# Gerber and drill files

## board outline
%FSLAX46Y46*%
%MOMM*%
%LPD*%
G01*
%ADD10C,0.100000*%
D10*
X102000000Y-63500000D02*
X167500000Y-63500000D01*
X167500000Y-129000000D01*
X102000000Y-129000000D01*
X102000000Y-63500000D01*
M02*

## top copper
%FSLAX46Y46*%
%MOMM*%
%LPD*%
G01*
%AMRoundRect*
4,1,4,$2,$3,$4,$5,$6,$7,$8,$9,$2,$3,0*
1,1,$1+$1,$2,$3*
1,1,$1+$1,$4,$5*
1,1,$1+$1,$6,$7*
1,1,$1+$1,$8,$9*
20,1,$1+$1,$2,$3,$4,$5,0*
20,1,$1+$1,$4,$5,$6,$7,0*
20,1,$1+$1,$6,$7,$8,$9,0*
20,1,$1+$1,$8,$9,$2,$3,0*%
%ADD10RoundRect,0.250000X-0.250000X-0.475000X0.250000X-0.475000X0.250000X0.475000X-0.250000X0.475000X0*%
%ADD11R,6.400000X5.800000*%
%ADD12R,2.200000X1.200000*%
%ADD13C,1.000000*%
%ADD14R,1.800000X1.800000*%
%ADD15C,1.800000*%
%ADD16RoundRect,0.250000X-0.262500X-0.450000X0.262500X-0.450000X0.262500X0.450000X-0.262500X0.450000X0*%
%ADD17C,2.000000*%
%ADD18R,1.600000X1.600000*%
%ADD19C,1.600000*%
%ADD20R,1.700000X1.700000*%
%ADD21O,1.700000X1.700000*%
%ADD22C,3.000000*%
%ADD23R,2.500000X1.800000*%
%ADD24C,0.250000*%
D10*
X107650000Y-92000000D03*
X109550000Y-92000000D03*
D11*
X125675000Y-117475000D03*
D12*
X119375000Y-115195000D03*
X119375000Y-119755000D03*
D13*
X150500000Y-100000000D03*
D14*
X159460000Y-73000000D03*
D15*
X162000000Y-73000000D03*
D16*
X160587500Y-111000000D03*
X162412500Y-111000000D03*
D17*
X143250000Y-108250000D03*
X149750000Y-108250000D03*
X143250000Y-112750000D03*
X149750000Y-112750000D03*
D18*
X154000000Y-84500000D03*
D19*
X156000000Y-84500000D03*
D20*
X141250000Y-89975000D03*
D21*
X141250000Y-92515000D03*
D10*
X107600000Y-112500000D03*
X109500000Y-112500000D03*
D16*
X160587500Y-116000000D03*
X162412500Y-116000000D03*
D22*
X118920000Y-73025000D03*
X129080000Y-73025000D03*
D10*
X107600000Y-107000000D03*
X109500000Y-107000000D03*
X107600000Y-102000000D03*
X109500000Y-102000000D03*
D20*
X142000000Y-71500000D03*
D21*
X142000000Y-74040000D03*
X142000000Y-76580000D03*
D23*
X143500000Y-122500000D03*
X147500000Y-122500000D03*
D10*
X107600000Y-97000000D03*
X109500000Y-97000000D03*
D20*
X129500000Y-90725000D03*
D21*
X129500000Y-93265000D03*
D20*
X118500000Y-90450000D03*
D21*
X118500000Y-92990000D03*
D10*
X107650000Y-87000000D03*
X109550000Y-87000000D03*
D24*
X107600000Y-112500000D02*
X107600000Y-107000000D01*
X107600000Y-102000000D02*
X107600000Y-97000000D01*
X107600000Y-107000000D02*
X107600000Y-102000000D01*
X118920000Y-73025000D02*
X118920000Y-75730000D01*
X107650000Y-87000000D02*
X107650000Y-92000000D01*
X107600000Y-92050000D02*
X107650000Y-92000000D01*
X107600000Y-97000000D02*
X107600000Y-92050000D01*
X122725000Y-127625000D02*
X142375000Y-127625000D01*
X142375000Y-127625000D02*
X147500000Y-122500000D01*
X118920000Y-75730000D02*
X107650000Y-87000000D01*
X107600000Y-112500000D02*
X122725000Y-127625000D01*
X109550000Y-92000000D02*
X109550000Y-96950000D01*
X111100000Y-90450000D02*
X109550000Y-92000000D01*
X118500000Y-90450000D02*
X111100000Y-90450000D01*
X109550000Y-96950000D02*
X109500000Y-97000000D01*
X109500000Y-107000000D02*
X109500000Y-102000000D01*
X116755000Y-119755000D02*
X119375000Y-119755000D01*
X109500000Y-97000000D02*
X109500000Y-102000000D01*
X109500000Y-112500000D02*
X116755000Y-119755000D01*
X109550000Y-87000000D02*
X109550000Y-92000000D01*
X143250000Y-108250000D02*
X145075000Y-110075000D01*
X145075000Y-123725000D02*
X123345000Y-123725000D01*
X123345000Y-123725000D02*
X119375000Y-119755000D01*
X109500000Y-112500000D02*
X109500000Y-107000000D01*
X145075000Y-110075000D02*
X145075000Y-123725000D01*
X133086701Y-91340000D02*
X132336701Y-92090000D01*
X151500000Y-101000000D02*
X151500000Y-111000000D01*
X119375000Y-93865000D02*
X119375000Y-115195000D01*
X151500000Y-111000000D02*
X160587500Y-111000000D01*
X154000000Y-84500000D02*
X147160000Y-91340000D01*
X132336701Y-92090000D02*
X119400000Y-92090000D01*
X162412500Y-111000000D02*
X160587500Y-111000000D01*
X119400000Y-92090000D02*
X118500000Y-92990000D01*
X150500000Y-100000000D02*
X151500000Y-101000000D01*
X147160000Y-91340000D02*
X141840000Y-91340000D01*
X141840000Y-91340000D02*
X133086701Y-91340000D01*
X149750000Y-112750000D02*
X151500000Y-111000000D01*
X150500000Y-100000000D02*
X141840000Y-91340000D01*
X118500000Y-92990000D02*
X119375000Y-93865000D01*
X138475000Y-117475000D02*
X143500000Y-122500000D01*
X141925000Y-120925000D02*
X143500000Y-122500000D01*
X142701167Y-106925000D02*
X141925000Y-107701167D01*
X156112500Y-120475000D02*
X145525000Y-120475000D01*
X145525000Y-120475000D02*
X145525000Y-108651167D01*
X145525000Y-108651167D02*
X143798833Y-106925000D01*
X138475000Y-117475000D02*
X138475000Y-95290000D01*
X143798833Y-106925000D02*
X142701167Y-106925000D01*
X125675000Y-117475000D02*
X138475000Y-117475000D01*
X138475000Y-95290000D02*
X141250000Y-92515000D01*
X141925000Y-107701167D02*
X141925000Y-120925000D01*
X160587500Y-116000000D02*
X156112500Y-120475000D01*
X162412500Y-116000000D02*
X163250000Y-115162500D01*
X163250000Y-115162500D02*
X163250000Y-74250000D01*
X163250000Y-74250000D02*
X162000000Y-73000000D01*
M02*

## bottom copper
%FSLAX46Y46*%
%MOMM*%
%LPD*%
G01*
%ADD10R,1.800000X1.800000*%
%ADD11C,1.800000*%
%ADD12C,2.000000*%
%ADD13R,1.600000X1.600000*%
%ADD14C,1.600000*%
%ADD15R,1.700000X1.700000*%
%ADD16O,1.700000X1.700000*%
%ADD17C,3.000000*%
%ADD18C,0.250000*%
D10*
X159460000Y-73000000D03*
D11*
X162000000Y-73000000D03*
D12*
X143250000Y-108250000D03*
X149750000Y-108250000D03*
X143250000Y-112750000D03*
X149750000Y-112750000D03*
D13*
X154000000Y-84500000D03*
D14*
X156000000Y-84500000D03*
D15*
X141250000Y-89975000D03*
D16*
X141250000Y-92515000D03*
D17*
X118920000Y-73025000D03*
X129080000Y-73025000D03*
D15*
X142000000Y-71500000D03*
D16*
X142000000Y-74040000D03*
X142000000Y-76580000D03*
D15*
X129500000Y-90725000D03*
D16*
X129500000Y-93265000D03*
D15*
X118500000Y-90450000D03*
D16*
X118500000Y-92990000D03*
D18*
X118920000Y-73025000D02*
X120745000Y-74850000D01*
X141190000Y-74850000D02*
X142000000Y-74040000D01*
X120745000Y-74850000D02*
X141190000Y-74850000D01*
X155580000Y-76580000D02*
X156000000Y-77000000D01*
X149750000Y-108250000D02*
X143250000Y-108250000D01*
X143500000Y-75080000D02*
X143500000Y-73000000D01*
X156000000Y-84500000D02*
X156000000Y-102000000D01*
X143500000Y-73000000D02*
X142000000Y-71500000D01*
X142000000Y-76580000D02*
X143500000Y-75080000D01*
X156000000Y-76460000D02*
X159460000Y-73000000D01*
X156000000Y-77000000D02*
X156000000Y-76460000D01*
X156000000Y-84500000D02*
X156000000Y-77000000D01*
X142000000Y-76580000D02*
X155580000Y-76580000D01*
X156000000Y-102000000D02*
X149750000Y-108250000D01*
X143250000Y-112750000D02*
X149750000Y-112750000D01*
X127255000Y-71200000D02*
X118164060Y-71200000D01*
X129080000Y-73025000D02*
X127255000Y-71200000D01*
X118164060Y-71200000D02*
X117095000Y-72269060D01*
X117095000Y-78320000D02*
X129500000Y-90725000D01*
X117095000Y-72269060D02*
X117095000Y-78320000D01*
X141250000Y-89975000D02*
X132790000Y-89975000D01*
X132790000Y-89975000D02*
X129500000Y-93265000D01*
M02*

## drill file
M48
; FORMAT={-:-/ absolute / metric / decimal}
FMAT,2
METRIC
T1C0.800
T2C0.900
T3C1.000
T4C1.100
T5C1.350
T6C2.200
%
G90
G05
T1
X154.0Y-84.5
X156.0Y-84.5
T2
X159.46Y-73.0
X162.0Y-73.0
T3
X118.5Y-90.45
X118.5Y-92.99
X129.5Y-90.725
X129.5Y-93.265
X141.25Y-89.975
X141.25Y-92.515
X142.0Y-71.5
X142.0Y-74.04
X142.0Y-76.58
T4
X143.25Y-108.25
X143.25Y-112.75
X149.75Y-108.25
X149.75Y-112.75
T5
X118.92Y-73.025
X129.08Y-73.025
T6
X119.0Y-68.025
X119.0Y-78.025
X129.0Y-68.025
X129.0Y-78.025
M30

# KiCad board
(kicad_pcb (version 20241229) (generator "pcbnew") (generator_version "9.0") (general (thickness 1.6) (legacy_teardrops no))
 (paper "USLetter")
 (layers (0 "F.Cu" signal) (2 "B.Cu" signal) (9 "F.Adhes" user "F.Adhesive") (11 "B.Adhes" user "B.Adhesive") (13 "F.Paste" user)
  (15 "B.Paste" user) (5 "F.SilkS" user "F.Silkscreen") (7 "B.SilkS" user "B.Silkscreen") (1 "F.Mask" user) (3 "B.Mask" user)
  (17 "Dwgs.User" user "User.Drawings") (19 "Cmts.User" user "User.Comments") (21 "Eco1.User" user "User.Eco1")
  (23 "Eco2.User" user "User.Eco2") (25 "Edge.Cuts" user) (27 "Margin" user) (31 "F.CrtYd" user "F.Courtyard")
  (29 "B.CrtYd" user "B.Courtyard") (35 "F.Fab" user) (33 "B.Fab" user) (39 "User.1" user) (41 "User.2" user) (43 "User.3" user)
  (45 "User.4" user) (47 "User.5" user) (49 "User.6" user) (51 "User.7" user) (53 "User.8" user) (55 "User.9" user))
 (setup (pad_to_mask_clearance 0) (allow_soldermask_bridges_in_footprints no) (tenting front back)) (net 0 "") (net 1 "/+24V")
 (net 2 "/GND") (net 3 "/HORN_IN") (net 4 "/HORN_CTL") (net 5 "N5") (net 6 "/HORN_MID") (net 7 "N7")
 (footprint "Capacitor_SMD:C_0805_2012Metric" (layer "F.Cu") (at 108.6 92)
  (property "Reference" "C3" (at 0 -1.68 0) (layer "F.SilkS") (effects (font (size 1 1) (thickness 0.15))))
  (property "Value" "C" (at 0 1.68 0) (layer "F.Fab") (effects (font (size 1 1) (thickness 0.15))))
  (pad "1" smd roundrect (at -0.95 0) (size 1 1.45) (layers "F.Cu" "F.Mask" "F.Paste") (roundrect_rratio 0.25) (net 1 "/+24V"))
  (pad "2" smd roundrect (at 0.95 0) (size 1 1.45) (layers "F.Cu" "F.Mask" "F.Paste") (roundrect_rratio 0.25) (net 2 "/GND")))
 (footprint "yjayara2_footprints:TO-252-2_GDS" (layer "F.Cu") (at 123.575 117.475)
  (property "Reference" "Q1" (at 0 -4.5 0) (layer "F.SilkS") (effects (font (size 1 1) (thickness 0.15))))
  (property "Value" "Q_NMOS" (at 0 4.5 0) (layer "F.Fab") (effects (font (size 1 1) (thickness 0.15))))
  (pad "" smd rect (at 0.425 -1.525) (size 3.05 2.75) (layers "F.Paste"))
  (pad "" smd rect (at 0.425 1.525) (size 3.05 2.75) (layers "F.Paste"))
  (pad "" smd rect (at 3.775 -1.525) (size 3.05 2.75) (layers "F.Paste"))
  (pad "" smd rect (at 3.775 1.525) (size 3.05 2.75) (layers "F.Paste"))
  (pad "D" smd rect (at 2.1 0) (size 6.4 5.8) (layers "F.Cu" "F.Mask") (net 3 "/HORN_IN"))
  (pad "G" smd rect (at -4.2 -2.28) (size 2.2 1.2) (layers "F.Cu" "F.Mask" "F.Paste") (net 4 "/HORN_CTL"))
  (pad "S" smd rect (at -4.2 2.28) (size 2.2 1.2) (layers "F.Cu" "F.Mask" "F.Paste") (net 2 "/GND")))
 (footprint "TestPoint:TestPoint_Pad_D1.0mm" (layer "F.Cu") (at 150.5 100)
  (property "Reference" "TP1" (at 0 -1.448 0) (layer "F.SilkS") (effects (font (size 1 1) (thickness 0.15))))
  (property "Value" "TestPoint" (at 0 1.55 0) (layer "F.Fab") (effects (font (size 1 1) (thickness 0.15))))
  (pad "1" smd circle (at 0 0) (size 1 1) (layers "F.Cu" "F.Mask") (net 4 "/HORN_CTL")))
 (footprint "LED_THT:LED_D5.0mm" (layer "F.Cu") (at 159.46 73)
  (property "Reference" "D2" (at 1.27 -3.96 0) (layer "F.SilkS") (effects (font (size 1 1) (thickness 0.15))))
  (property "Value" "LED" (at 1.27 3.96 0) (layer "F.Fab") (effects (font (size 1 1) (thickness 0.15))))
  (pad "1" thru_hole rect (at 0 0) (size 1.8 1.8) (drill 0.9) (layers "*.Cu" "*.Mask") (remove_unused_layers no) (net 2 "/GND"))
  (pad "2" thru_hole circle (at 2.54 0) (size 1.8 1.8) (drill 0.9) (layers "*.Cu" "*.Mask") (remove_unused_layers no) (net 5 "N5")))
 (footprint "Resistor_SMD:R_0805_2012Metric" (layer "F.Cu") (at 161.5 111)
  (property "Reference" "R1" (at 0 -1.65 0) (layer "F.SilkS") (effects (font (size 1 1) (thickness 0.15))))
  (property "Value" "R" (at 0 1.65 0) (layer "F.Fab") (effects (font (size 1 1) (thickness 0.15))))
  (pad "1" smd roundrect (at -0.9125 0) (size 1.025 1.4) (layers "F.Cu" "F.Mask" "F.Paste") (roundrect_rratio 0.243902) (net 4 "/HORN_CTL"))
  (pad "2" smd roundrect (at 0.9125 0) (size 1.025 1.4) (layers "F.Cu" "F.Mask" "F.Paste") (roundrect_rratio 0.243902) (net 4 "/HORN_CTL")))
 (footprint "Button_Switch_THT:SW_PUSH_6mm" (layer "F.Cu") (at 143.25 108.25)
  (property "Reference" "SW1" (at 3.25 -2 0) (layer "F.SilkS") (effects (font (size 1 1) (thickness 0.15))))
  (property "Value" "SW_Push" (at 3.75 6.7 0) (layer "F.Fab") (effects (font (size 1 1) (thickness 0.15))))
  (pad "1" thru_hole circle (at 0 0 90) (size 2 2) (drill 1.1) (layers "*.Cu" "*.Mask") (remove_unused_layers no) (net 2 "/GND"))
  (pad "1" thru_hole circle (at 6.5 0 90) (size 2 2) (drill 1.1) (layers "*.Cu" "*.Mask") (remove_unused_layers no) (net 2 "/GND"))
  (pad "2" thru_hole circle (at 0 4.5 90) (size 2 2) (drill 1.1) (layers "*.Cu" "*.Mask") (remove_unused_layers no) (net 4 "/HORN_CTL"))
  (pad "2" thru_hole circle (at 6.5 4.5 90) (size 2 2) (drill 1.1) (layers "*.Cu" "*.Mask") (remove_unused_layers no) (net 4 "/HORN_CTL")))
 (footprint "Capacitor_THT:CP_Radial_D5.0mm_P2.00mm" (layer "F.Cu") (at 154 84.5)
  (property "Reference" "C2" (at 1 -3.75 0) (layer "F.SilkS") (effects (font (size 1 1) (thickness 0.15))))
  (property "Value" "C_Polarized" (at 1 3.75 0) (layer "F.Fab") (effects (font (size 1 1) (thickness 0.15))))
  (pad "1" thru_hole rect (at 0 0) (size 1.6 1.6) (drill 0.8) (layers "*.Cu" "*.Mask") (remove_unused_layers no) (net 4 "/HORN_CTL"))
  (pad "2" thru_hole circle (at 2 0) (size 1.6 1.6) (drill 0.8) (layers "*.Cu" "*.Mask") (remove_unused_layers no) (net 2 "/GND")))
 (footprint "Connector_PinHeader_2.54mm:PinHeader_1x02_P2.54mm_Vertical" (layer "F.Cu") (at 141.25 89.975)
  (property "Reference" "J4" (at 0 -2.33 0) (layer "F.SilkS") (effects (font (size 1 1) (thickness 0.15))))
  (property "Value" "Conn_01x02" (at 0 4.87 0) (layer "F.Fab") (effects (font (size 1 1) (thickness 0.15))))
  (pad "1" thru_hole rect (at 0 0) (size 1.7 1.7) (drill 1) (layers "*.Cu" "*.Mask") (remove_unused_layers no) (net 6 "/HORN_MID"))
  (pad "2" thru_hole oval (at 0 2.54) (size 1.7 1.7) (drill 1) (layers "*.Cu" "*.Mask") (remove_unused_layers no) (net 3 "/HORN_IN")))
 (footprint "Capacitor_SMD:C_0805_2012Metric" (layer "F.Cu") (at 108.55 112.5)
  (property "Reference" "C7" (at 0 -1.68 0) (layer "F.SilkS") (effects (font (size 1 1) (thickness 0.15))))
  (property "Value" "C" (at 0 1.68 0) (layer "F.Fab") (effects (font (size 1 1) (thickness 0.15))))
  (pad "1" smd roundrect (at -0.95 0) (size 1 1.45) (layers "F.Cu" "F.Mask" "F.Paste") (roundrect_rratio 0.25) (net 1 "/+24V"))
  (pad "2" smd roundrect (at 0.95 0) (size 1 1.45) (layers "F.Cu" "F.Mask" "F.Paste") (roundrect_rratio 0.25) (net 2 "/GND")))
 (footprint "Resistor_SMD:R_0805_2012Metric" (layer "F.Cu") (at 161.5 116)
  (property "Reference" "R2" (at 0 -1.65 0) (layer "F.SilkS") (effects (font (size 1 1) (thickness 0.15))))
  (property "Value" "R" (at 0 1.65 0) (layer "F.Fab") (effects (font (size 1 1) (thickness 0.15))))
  (pad "1" smd roundrect (at -0.9125 0) (size 1.025 1.4) (layers "F.Cu" "F.Mask" "F.Paste") (roundrect_rratio 0.243902) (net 3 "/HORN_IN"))
  (pad "2" smd roundrect (at 0.9125 0) (size 1.025 1.4) (layers "F.Cu" "F.Mask" "F.Paste") (roundrect_rratio 0.243902) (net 5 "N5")))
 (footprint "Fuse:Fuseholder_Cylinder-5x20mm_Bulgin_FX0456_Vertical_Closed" (layer "F.Cu") (at 118.92 73.025)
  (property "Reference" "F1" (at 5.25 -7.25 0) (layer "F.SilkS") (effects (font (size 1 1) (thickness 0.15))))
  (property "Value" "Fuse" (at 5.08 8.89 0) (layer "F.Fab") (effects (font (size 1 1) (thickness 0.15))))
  (pad "" np_thru_hole circle (at 0.08 -5) (size 2.2 2.2) (drill 2.2) (layers "*.Cu" "*.Mask"))
  (pad "" np_thru_hole circle (at 0.08 5) (size 2.2 2.2) (drill 2.2) (layers "*.Cu" "*.Mask"))
  (pad "" np_thru_hole circle (at 10.08 -5) (size 2.2 2.2) (drill 2.2) (layers "*.Cu" "*.Mask"))
  (pad "" np_thru_hole circle (at 10.08 5) (size 2.2 2.2) (drill 2.2) (layers "*.Cu" "*.Mask"))
  (pad "1" thru_hole circle (at 0 0) (size 3 3) (drill 1.35) (layers "*.Cu" "*.Mask") (remove_unused_layers no) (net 1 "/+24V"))
  (pad "2" thru_hole circle (at 10.16 0) (size 3 3) (drill 1.35) (layers "*.Cu" "*.Mask") (remove_unused_layers no) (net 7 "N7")))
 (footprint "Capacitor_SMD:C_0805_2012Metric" (layer "F.Cu") (at 108.55 107)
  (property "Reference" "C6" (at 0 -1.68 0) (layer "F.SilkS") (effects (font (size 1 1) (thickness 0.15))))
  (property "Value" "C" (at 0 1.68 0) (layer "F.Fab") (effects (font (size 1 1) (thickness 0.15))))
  (pad "1" smd roundrect (at -0.95 0) (size 1 1.45) (layers "F.Cu" "F.Mask" "F.Paste") (roundrect_rratio 0.25) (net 1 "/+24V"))
  (pad "2" smd roundrect (at 0.95 0) (size 1 1.45) (layers "F.Cu" "F.Mask" "F.Paste") (roundrect_rratio 0.25) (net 2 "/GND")))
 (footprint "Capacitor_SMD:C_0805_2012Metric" (layer "F.Cu") (at 108.55 102)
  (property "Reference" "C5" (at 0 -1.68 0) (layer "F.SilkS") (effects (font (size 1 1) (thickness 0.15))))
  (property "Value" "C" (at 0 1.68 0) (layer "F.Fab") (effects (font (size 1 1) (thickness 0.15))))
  (pad "1" smd roundrect (at -0.95 0) (size 1 1.45) (layers "F.Cu" "F.Mask" "F.Paste") (roundrect_rratio 0.25) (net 1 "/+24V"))
  (pad "2" smd roundrect (at 0.95 0) (size 1 1.45) (layers "F.Cu" "F.Mask" "F.Paste") (roundrect_rratio 0.25) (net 2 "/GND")))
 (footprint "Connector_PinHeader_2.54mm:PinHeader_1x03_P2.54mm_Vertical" (layer "F.Cu") (at 142 71.5)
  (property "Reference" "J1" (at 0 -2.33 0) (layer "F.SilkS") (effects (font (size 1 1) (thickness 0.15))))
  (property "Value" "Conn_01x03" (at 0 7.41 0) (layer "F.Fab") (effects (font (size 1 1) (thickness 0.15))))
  (pad "1" thru_hole rect (at 0 0) (size 1.7 1.7) (drill 1) (layers "*.Cu" "*.Mask") (remove_unused_layers no) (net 2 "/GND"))
  (pad "2" thru_hole oval (at 0 2.54) (size 1.7 1.7) (drill 1) (layers "*.Cu" "*.Mask") (remove_unused_layers no) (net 1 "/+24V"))
  (pad "3" thru_hole oval (at 0 5.08) (size 1.7 1.7) (drill 1) (layers "*.Cu" "*.Mask") (remove_unused_layers no) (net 2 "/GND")))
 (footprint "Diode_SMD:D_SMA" (layer "F.Cu") (at 145.5 122.5)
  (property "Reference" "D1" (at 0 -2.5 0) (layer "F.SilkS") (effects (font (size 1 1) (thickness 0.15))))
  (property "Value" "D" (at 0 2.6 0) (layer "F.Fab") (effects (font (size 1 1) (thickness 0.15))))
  (pad "1" smd rect (at -2 0) (size 2.5 1.8) (layers "F.Cu" "F.Mask" "F.Paste") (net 3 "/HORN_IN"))
  (pad "2" smd rect (at 2 0) (size 2.5 1.8) (layers "F.Cu" "F.Mask" "F.Paste") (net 1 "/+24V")))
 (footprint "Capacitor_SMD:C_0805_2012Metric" (layer "F.Cu") (at 108.55 97)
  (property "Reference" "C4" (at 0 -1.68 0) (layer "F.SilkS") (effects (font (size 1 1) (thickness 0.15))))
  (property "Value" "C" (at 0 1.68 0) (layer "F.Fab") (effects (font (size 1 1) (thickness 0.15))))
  (pad "1" smd roundrect (at -0.95 0) (size 1 1.45) (layers "F.Cu" "F.Mask" "F.Paste") (roundrect_rratio 0.25) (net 1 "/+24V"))
  (pad "2" smd roundrect (at 0.95 0) (size 1 1.45) (layers "F.Cu" "F.Mask" "F.Paste") (roundrect_rratio 0.25) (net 2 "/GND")))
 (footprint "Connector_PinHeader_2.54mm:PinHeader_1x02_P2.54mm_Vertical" (layer "F.Cu") (at 129.5 90.725)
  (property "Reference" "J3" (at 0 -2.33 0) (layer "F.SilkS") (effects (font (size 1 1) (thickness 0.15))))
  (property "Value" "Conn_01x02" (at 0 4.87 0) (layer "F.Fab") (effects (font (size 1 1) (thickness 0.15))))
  (pad "1" thru_hole rect (at 0 0) (size 1.7 1.7) (drill 1) (layers "*.Cu" "*.Mask") (remove_unused_layers no) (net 7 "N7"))
  (pad "2" thru_hole oval (at 0 2.54) (size 1.7 1.7) (drill 1) (layers "*.Cu" "*.Mask") (remove_unused_layers no) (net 6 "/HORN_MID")))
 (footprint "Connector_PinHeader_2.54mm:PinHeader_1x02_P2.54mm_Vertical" (layer "F.Cu") (at 118.5 90.45)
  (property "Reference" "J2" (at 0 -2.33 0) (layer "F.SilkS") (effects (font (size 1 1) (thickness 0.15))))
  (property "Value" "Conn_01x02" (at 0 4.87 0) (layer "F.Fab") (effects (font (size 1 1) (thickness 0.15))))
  (pad "1" thru_hole rect (at 0 0) (size 1.7 1.7) (drill 1) (layers "*.Cu" "*.Mask") (remove_unused_layers no) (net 2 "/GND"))
  (pad "2" thru_hole oval (at 0 2.54) (size 1.7 1.7) (drill 1) (layers "*.Cu" "*.Mask") (remove_unused_layers no) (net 4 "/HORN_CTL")))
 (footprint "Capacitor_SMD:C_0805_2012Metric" (layer "F.Cu") (at 108.6 87)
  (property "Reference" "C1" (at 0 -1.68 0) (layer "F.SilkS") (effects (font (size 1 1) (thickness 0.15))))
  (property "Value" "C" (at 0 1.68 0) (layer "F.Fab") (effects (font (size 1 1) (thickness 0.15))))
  (pad "1" smd roundrect (at -0.95 0) (size 1 1.45) (layers "F.Cu" "F.Mask" "F.Paste") (roundrect_rratio 0.25) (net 1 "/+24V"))
  (pad "2" smd roundrect (at 0.95 0) (size 1 1.45) (layers "F.Cu" "F.Mask" "F.Paste") (roundrect_rratio 0.25) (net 2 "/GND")))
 (gr_rect (start 102 63.5) (end 167.5 129) (stroke (width 0.1) (type default)) (fill no) (layer "Edge.Cuts"))
 (segment (start 107.6 112.5) (end 107.6 107) (width 0.25) (layer "F.Cu") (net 1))
 (segment (start 107.6 102) (end 107.6 97) (width 0.25) (layer "F.Cu") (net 1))
 (segment (start 107.6 107) (end 107.6 102) (width 0.25) (layer "F.Cu") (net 1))
 (segment (start 118.92 73.025) (end 118.92 75.73) (width 0.25) (layer "F.Cu") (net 1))
 (segment (start 107.65 87) (end 107.65 92) (width 0.25) (layer "F.Cu") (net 1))
 (segment (start 107.6 92.05) (end 107.65 92) (width 0.25) (layer "F.Cu") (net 1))
 (segment (start 107.6 97) (end 107.6 92.05) (width 0.25) (layer "F.Cu") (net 1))
 (segment (start 122.725 127.625) (end 142.375 127.625) (width 0.25) (layer "F.Cu") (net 1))
 (segment (start 142.375 127.625) (end 147.5 122.5) (width 0.25) (layer "F.Cu") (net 1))
 (segment (start 118.92 75.73) (end 107.65 87) (width 0.25) (layer "F.Cu") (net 1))
 (segment (start 107.6 112.5) (end 122.725 127.625) (width 0.25) (layer "F.Cu") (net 1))
 (segment (start 118.92 73.025) (end 120.745 74.85) (width 0.25) (layer "B.Cu") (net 1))
 (segment (start 141.19 74.85) (end 142 74.04) (width 0.25) (layer "B.Cu") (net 1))
 (segment (start 120.745 74.85) (end 141.19 74.85) (width 0.25) (layer "B.Cu") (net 1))
 (segment (start 109.55 92) (end 109.55 96.95) (width 0.25) (layer "F.Cu") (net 2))
 (segment (start 111.1 90.45) (end 109.55 92) (width 0.25) (layer "F.Cu") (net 2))
 (segment (start 118.5 90.45) (end 111.1 90.45) (width 0.25) (layer "F.Cu") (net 2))
 (segment (start 109.55 96.95) (end 109.5 97) (width 0.25) (layer "F.Cu") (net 2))
 (segment (start 109.5 107) (end 109.5 102) (width 0.25) (layer "F.Cu") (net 2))
 (segment (start 116.755 119.755) (end 119.375 119.755) (width 0.25) (layer "F.Cu") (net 2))
 (segment (start 109.5 97) (end 109.5 102) (width 0.25) (layer "F.Cu") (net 2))
 (segment (start 109.5 112.5) (end 116.755 119.755) (width 0.25) (layer "F.Cu") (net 2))
 (segment (start 109.55 87) (end 109.55 92) (width 0.25) (layer "F.Cu") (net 2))
 (segment (start 143.25 108.25) (end 145.075 110.075) (width 0.25) (layer "F.Cu") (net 2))
 (segment (start 145.075 123.725) (end 123.345 123.725) (width 0.25) (layer "F.Cu") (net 2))
 (segment (start 123.345 123.725) (end 119.375 119.755) (width 0.25) (layer "F.Cu") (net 2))
 (segment (start 109.5 112.5) (end 109.5 107) (width 0.25) (layer "F.Cu") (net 2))
 (segment (start 145.075 110.075) (end 145.075 123.725) (width 0.25) (layer "F.Cu") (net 2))
 (segment (start 155.58 76.58) (end 156 77) (width 0.25) (layer "B.Cu") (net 2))
 (segment (start 149.75 108.25) (end 143.25 108.25) (width 0.25) (layer "B.Cu") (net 2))
 (segment (start 143.5 75.08) (end 143.5 73) (width 0.25) (layer "B.Cu") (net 2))
 (segment (start 156 84.5) (end 156 102) (width 0.25) (layer "B.Cu") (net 2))
 (segment (start 143.5 73) (end 142 71.5) (width 0.25) (layer "B.Cu") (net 2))
 (segment (start 142 76.58) (end 143.5 75.08) (width 0.25) (layer "B.Cu") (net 2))
 (segment (start 156 76.46) (end 159.46 73) (width 0.25) (layer "B.Cu") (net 2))
 (segment (start 156 77) (end 156 76.46) (width 0.25) (layer "B.Cu") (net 2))
 (segment (start 156 84.5) (end 156 77) (width 0.25) (layer "B.Cu") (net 2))
 (segment (start 142 76.58) (end 155.58 76.58) (width 0.25) (layer "B.Cu") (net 2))
 (segment (start 156 102) (end 149.75 108.25) (width 0.25) (layer "B.Cu") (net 2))
 (segment (start 133.086701 91.34) (end 132.336701 92.09) (width 0.25) (layer "F.Cu") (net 4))
 (segment (start 151.5 101) (end 151.5 111) (width 0.25) (layer "F.Cu") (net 4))
 (segment (start 119.375 93.865) (end 119.375 115.195) (width 0.25) (layer "F.Cu") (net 4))
 (segment (start 151.5 111) (end 160.5875 111) (width 0.25) (layer "F.Cu") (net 4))
 (segment (start 154 84.5) (end 147.16 91.34) (width 0.25) (layer "F.Cu") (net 4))
 (segment (start 132.336701 92.09) (end 119.4 92.09) (width 0.25) (layer "F.Cu") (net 4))
 (segment (start 162.4125 111) (end 160.5875 111) (width 0.25) (layer "F.Cu") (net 4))
 (segment (start 119.4 92.09) (end 118.5 92.99) (width 0.25) (layer "F.Cu") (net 4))
 (segment (start 150.5 100) (end 151.5 101) (width 0.25) (layer "F.Cu") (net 4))
 (segment (start 147.16 91.34) (end 141.84 91.34) (width 0.25) (layer "F.Cu") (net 4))
 (segment (start 141.84 91.34) (end 133.086701 91.34) (width 0.25) (layer "F.Cu") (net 4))
 (segment (start 149.75 112.75) (end 151.5 111) (width 0.25) (layer "F.Cu") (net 4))
 (segment (start 150.5 100) (end 141.84 91.34) (width 0.25) (layer "F.Cu") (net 4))
 (segment (start 118.5 92.99) (end 119.375 93.865) (width 0.25) (layer "F.Cu") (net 4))
 (segment (start 143.25 112.75) (end 149.75 112.75) (width 0.25) (layer "B.Cu") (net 4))
 (segment (start 138.475 117.475) (end 143.5 122.5) (width 0.25) (layer "F.Cu") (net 3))
 (segment (start 141.925 120.925) (end 143.5 122.5) (width 0.25) (layer "F.Cu") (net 3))
 (segment (start 142.701167 106.925) (end 141.925 107.701167) (width 0.25) (layer "F.Cu") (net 3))
 (segment (start 156.1125 120.475) (end 145.525 120.475) (width 0.25) (layer "F.Cu") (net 3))
 (segment (start 145.525 120.475) (end 145.525 108.651167) (width 0.25) (layer "F.Cu") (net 3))
 (segment (start 145.525 108.651167) (end 143.798833 106.925) (width 0.25) (layer "F.Cu") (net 3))
 (segment (start 138.475 117.475) (end 138.475 95.29) (width 0.25) (layer "F.Cu") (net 3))
 (segment (start 143.798833 106.925) (end 142.701167 106.925) (width 0.25) (layer "F.Cu") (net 3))
 (segment (start 125.675 117.475) (end 138.475 117.475) (width 0.25) (layer "F.Cu") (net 3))
 (segment (start 138.475 95.29) (end 141.25 92.515) (width 0.25) (layer "F.Cu") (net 3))
 (segment (start 141.925 107.701167) (end 141.925 120.925) (width 0.25) (layer "F.Cu") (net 3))
 (segment (start 160.5875 116) (end 156.1125 120.475) (width 0.25) (layer "F.Cu") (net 3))
 (segment (start 162.4125 116) (end 163.25 115.1625) (width 0.25) (layer "F.Cu") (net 5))
 (segment (start 163.25 115.1625) (end 163.25 74.25) (width 0.25) (layer "F.Cu") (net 5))
 (segment (start 163.25 74.25) (end 162 73) (width 0.25) (layer "F.Cu") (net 5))
 (segment (start 127.255 71.2) (end 118.16406 71.2) (width 0.25) (layer "B.Cu") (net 7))
 (segment (start 129.08 73.025) (end 127.255 71.2) (width 0.25) (layer "B.Cu") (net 7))
 (segment (start 118.16406 71.2) (end 117.095 72.26906) (width 0.25) (layer "B.Cu") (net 7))
 (segment (start 117.095 78.32) (end 129.5 90.725) (width 0.25) (layer "B.Cu") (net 7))
 (segment (start 117.095 72.26906) (end 117.095 78.32) (width 0.25) (layer "B.Cu") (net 7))
 (segment (start 141.25 89.975) (end 132.79 89.975) (width 0.25) (layer "B.Cu") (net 6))
 (segment (start 132.79 89.975) (end 129.5 93.265) (width 0.25) (layer "B.Cu") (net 6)))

